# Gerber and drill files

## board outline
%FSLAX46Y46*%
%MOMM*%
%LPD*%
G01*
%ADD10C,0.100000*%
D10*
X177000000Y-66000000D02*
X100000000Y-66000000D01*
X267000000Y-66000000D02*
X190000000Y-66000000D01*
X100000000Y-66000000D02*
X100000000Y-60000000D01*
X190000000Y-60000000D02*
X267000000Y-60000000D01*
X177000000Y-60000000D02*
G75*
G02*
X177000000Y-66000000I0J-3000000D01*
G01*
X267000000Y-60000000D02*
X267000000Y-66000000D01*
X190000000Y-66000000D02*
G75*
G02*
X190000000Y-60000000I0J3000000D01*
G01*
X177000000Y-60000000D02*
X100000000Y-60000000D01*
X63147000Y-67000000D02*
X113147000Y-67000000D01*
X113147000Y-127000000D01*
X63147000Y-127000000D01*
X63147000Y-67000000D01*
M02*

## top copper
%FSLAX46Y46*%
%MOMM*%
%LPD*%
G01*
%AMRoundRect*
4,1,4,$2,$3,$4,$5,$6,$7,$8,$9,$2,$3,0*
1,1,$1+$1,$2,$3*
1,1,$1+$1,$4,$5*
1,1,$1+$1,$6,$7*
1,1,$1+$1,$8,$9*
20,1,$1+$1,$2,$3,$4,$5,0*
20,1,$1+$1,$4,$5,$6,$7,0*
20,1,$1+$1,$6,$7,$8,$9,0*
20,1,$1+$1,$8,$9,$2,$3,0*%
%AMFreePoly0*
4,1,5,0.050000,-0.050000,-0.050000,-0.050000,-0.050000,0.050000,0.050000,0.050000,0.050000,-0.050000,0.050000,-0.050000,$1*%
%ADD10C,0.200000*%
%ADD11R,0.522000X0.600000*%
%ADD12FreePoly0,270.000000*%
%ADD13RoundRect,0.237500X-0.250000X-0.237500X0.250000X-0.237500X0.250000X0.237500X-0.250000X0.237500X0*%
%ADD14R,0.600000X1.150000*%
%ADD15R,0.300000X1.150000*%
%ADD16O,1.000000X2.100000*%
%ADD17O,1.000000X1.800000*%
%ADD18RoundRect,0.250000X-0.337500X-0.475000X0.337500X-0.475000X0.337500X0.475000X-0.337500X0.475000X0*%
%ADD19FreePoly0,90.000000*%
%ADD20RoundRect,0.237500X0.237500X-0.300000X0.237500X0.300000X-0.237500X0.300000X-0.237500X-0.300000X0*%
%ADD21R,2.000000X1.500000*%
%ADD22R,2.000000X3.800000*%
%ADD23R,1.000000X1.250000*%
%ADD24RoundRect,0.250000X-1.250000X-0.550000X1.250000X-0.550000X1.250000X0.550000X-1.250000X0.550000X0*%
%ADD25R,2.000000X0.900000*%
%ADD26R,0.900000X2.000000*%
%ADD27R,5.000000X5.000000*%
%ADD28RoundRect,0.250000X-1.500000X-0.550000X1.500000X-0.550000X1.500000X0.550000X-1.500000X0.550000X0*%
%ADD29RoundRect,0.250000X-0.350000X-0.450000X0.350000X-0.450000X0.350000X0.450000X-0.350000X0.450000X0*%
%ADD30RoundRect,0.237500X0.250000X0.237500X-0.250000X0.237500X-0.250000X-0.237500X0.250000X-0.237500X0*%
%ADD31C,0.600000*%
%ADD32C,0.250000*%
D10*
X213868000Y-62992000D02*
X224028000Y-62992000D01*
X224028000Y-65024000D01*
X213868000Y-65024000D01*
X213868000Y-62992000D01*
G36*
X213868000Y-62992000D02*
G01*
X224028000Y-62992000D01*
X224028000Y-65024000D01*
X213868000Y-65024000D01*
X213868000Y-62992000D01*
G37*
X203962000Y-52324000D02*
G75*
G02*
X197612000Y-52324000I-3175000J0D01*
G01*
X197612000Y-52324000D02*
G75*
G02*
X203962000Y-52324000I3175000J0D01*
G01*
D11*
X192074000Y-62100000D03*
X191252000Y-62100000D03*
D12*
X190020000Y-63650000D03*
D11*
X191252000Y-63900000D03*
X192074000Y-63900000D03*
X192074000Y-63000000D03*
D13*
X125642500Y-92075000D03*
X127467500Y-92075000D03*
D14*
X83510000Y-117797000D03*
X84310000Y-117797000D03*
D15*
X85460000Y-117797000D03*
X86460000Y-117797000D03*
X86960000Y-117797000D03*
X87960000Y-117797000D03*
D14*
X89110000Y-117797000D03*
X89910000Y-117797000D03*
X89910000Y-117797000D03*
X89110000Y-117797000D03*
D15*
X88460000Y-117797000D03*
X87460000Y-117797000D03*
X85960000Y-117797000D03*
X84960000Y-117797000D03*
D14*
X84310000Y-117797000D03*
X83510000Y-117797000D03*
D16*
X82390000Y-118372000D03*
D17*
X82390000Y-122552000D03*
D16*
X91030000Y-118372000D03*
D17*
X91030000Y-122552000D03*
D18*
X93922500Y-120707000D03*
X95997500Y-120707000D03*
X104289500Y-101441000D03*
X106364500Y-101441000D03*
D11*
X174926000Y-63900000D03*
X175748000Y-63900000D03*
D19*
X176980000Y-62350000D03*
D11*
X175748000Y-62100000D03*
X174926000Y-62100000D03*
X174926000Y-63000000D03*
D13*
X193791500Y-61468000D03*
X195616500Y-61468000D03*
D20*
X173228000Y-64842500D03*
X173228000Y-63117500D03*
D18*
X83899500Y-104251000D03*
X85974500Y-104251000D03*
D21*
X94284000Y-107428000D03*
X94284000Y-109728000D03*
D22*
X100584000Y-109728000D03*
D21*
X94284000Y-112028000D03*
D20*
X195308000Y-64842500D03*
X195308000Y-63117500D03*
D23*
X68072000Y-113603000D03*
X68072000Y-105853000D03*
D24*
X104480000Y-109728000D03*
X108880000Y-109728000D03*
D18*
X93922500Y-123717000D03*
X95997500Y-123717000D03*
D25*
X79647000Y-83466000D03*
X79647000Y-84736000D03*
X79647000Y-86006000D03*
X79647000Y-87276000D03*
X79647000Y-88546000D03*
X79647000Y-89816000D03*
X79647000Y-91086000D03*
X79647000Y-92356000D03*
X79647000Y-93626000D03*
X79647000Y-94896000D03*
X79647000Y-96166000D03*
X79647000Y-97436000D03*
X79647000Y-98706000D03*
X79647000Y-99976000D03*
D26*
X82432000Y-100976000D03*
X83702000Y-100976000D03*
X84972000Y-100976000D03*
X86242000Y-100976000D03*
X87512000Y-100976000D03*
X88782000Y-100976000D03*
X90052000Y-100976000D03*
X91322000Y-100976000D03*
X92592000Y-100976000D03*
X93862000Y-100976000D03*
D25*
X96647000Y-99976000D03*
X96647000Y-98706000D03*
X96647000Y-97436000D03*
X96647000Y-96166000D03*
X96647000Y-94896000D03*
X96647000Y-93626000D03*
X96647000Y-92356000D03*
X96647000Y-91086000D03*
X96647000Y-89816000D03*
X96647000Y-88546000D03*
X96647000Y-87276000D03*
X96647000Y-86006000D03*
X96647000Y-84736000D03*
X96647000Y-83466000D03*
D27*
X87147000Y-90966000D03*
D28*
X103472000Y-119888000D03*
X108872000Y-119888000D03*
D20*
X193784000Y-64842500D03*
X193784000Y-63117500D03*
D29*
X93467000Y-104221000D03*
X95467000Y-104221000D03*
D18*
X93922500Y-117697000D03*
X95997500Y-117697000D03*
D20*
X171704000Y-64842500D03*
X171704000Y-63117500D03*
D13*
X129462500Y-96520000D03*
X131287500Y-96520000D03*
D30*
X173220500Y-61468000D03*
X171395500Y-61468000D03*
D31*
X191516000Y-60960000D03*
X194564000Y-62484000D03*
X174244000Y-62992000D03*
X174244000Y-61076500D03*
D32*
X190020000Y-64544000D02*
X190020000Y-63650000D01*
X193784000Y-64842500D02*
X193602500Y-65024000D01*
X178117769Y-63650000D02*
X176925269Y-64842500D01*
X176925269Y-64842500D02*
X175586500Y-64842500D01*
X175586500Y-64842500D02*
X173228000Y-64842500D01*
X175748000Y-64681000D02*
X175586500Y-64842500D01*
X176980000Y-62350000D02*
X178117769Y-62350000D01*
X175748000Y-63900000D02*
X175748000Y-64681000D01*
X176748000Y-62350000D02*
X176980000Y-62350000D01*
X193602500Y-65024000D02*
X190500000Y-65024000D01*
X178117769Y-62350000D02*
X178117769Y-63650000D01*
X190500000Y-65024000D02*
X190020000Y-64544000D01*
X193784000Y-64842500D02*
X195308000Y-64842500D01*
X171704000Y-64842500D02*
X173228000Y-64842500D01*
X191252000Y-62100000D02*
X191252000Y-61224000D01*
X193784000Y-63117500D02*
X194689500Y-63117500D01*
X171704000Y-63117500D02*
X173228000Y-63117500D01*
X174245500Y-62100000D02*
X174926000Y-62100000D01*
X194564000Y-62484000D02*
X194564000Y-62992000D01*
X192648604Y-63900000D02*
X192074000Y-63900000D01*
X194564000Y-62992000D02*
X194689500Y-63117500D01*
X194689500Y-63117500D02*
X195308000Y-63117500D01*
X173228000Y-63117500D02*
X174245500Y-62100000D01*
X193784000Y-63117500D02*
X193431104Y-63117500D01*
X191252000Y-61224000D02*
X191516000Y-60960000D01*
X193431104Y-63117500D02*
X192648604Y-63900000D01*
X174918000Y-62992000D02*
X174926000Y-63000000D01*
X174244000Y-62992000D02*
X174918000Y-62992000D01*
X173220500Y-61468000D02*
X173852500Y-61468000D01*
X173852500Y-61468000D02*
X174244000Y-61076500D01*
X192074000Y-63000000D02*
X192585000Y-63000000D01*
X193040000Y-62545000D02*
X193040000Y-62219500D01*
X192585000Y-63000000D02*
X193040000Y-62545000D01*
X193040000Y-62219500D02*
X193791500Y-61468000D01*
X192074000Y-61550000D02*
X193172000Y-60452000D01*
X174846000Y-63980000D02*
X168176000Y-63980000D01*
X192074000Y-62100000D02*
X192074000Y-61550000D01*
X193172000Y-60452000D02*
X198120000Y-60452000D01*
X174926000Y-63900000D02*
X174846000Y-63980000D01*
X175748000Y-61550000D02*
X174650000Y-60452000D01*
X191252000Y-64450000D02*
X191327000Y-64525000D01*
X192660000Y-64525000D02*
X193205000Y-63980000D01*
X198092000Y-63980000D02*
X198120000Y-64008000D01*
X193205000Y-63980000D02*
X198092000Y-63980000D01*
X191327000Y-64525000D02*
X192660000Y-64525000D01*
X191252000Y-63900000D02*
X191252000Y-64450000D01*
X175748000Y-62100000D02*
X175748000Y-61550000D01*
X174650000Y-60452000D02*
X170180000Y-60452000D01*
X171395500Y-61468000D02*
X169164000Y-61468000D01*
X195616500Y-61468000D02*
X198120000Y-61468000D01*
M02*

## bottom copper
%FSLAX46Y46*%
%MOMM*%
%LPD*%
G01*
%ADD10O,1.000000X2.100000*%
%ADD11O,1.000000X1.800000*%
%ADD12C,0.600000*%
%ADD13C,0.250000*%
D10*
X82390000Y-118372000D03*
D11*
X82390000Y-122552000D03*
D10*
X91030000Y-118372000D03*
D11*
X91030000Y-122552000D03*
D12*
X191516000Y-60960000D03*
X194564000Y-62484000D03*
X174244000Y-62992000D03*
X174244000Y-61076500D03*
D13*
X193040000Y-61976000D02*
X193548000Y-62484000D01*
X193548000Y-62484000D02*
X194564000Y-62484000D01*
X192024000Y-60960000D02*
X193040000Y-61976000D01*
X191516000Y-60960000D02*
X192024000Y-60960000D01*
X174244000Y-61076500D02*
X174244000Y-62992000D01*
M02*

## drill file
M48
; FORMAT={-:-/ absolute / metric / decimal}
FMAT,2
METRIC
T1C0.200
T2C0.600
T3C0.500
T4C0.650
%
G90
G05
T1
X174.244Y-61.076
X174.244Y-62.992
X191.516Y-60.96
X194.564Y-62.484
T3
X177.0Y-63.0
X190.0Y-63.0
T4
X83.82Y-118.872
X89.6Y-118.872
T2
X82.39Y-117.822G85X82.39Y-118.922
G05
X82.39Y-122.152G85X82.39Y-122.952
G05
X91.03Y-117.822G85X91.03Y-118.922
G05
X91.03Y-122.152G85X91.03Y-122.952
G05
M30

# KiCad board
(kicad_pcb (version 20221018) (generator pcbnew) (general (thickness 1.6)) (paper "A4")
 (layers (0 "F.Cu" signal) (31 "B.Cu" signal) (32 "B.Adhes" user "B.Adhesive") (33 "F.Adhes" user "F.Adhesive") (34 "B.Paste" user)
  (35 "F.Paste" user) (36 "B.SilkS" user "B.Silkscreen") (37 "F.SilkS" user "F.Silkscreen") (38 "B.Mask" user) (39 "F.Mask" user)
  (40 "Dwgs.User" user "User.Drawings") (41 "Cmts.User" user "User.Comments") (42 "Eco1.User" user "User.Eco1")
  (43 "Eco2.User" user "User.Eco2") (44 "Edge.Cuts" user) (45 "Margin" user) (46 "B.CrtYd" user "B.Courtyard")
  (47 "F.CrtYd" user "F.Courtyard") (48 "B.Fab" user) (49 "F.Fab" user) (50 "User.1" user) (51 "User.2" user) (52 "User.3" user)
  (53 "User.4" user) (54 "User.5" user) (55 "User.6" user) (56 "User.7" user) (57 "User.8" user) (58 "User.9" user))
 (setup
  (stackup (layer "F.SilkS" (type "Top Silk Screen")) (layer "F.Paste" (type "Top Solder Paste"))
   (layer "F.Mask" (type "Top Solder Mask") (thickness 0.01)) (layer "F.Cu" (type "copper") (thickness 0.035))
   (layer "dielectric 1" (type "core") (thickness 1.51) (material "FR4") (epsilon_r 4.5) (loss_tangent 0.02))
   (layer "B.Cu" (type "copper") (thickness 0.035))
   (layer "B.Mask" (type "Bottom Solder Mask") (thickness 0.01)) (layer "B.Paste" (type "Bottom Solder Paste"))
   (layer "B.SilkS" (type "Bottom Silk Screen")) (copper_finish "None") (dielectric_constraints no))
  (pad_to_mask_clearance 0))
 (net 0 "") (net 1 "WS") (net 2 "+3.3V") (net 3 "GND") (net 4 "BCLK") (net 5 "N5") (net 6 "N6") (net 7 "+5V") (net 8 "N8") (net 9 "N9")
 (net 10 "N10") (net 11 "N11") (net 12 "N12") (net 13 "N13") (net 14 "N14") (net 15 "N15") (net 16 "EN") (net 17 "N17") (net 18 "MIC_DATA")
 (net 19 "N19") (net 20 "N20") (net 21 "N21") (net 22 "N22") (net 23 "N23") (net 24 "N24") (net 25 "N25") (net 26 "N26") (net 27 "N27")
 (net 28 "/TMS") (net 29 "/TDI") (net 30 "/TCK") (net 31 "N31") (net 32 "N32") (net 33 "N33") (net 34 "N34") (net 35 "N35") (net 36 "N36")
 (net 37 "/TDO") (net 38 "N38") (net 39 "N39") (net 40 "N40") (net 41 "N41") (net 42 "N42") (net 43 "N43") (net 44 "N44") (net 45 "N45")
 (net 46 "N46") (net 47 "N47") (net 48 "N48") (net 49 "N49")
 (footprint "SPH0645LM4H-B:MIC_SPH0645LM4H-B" (layer "F.Cu") (at 190 63 -90)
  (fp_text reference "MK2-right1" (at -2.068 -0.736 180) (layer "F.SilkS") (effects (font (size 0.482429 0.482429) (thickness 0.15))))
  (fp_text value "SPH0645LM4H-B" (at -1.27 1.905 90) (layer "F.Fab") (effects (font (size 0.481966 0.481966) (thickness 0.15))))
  (pad "" np_thru_hole circle (at 0 0 270) (size 0.5 0.5) (drill 0.5) (layers "*.Cu" "*.Mask"))
  (pad "1" smd rect (at -0.9 -2.074 270) (size 0.6 0.522) (layers "F.Cu" "F.Paste" "F.Mask") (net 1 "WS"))
  (pad "2" smd rect (at -0.9 -1.252 270) (size 0.6 0.522) (layers "F.Cu" "F.Paste" "F.Mask") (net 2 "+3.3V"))
  (pad "3" smd custom (at 0.65 -0.02 270) (size 0.1 0.1) (layers "F.Cu") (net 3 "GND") (zone_connect 0) (thermal_bridge_angle 45)
   (options (clearance outline) (anchor rect)) (primitives))
  (pad "4" smd rect (at 0.9 -1.252 270) (size 0.6 0.522) (layers "F.Cu" "F.Paste" "F.Mask") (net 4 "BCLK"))
  (pad "5" smd rect (at 0.9 -2.074 270) (size 0.6 0.522) (layers "F.Cu" "F.Paste" "F.Mask") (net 2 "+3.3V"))
  (pad "6" smd rect (at 0 -2.074 270) (size 0.6 0.522) (layers "F.Cu" "F.Paste" "F.Mask") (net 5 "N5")))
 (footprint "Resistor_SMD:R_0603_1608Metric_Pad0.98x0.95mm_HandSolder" (layer "F.Cu") (at 126.555 92.075)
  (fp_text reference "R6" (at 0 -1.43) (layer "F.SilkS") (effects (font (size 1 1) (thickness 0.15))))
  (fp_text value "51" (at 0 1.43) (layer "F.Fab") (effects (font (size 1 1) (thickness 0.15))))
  (pad "1" smd roundrect (at -0.9125 0) (size 0.975 0.95) (layers "F.Cu" "F.Paste" "F.Mask") (roundrect_rratio 0.25) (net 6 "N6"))
  (pad "2" smd roundrect (at 0.9125 0) (size 0.975 0.95) (layers "F.Cu" "F.Paste" "F.Mask") (roundrect_rratio 0.25) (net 1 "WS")))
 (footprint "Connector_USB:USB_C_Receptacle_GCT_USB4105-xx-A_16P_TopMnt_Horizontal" (layer "F.Cu") (at 86.71 121.477)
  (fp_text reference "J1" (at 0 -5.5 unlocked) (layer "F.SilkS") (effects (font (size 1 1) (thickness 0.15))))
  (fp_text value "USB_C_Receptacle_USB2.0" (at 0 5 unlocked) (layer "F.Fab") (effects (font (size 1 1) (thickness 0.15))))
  (pad "" np_thru_hole circle (at -2.89 -2.605) (size 0.65 0.65) (drill 0.65) (layers "F&B.Cu" "*.Mask"))
  (pad "" np_thru_hole circle (at 2.89 -2.605) (size 0.65 0.65) (drill 0.65) (layers "F&B.Cu" "*.Mask"))
  (pad "A1" smd rect (at -3.2 -3.68) (size 0.6 1.15) (layers "F.Cu" "F.Paste" "F.Mask") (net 3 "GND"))
  (pad "A4" smd rect (at -2.4 -3.68) (size 0.6 1.15) (layers "F.Cu" "F.Paste" "F.Mask") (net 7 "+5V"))
  (pad "A5" smd rect (at -1.25 -3.68) (size 0.3 1.15) (layers "F.Cu" "F.Paste" "F.Mask") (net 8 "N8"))
  (pad "A6" smd rect (at -0.25 -3.68) (size 0.3 1.15) (layers "F.Cu" "F.Paste" "F.Mask") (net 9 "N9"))
  (pad "A7" smd rect (at 0.25 -3.68) (size 0.3 1.15) (layers "F.Cu" "F.Paste" "F.Mask") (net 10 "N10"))
  (pad "A8" smd rect (at 1.25 -3.68) (size 0.3 1.15) (layers "F.Cu" "F.Paste" "F.Mask") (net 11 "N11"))
  (pad "A9" smd rect (at 2.4 -3.68) (size 0.6 1.15) (layers "F.Cu" "F.Paste" "F.Mask") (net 7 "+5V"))
  (pad "A12" smd rect (at 3.2 -3.68) (size 0.6 1.15) (layers "F.Cu" "F.Paste" "F.Mask") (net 3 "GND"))
  (pad "B1" smd rect (at 3.2 -3.68) (size 0.6 1.15) (layers "F.Cu" "F.Paste" "F.Mask") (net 3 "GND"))
  (pad "B4" smd rect (at 2.4 -3.68) (size 0.6 1.15) (layers "F.Cu" "F.Paste" "F.Mask") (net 7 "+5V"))
  (pad "B5" smd rect (at 1.75 -3.68) (size 0.3 1.15) (layers "F.Cu" "F.Paste" "F.Mask") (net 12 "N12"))
  (pad "B6" smd rect (at 0.75 -3.68) (size 0.3 1.15) (layers "F.Cu" "F.Paste" "F.Mask") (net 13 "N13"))
  (pad "B7" smd rect (at -0.75 -3.68) (size 0.3 1.15) (layers "F.Cu" "F.Paste" "F.Mask") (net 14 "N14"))
  (pad "B8" smd rect (at -1.75 -3.68) (size 0.3 1.15) (layers "F.Cu" "F.Paste" "F.Mask") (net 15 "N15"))
  (pad "B9" smd rect (at -2.4 -3.68) (size 0.6 1.15) (layers "F.Cu" "F.Paste" "F.Mask") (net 7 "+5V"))
  (pad "B12" smd rect (at -3.2 -3.68) (size 0.6 1.15) (layers "F.Cu" "F.Paste" "F.Mask") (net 3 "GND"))
  (pad "S1" thru_hole oval (at -4.32 -3.105) (size 1 2.1) (drill oval 0.6 1.7) (layers "*.Cu" "*.Mask") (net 3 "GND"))
  (pad "S1" thru_hole oval (at -4.32 1.075) (size 1 1.8) (drill oval 0.6 1.4) (layers "*.Cu" "*.Mask") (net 3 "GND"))
  (pad "S1" thru_hole oval (at 4.32 -3.105) (size 1 2.1) (drill oval 0.6 1.7) (layers "*.Cu" "*.Mask") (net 3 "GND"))
  (pad "S1" thru_hole oval (at 4.32 1.075) (size 1 1.8) (drill oval 0.6 1.4) (layers "*.Cu" "*.Mask") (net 3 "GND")))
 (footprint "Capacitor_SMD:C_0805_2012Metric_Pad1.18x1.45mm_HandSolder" (layer "F.Cu") (at 94.96 120.707)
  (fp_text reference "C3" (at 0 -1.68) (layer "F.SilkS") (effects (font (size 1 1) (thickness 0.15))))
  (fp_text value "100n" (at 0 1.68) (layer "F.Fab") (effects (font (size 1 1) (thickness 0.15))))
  (pad "1" smd roundrect (at -1.0375 0) (size 1.175 1.45) (layers "F.Cu" "F.Paste" "F.Mask") (roundrect_rratio 0.212766) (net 3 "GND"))
  (pad "2" smd roundrect (at 1.0375 0) (size 1.175 1.45) (layers "F.Cu" "F.Paste" "F.Mask") (roundrect_rratio 0.212766) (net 2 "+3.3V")))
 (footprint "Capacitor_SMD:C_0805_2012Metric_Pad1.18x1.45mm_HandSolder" (layer "F.Cu") (at 105.327 101.441)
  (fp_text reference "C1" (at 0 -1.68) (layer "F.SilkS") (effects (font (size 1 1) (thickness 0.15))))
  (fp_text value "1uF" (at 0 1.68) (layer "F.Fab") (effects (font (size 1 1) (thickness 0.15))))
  (pad "1" smd roundrect (at -1.0375 0) (size 1.175 1.45) (layers "F.Cu" "F.Paste" "F.Mask") (roundrect_rratio 0.212766) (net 3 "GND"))
  (pad "2" smd roundrect (at 1.0375 0) (size 1.175 1.45) (layers "F.Cu" "F.Paste" "F.Mask") (roundrect_rratio 0.212766) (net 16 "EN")))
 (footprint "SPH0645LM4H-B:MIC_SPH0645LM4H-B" (layer "F.Cu") (at 177 63 90)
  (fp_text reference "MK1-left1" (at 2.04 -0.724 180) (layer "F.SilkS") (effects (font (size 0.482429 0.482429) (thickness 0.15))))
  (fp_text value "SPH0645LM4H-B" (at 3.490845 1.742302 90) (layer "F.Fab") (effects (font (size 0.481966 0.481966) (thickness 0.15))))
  (pad "" np_thru_hole circle (at 0 0 90) (size 0.5 0.5) (drill 0.5) (layers "*.Cu" "*.Mask"))
  (pad "1" smd rect (at -0.9 -2.074 90) (size 0.6 0.522) (layers "F.Cu" "F.Paste" "F.Mask") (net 1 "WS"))
  (pad "2" smd rect (at -0.9 -1.252 90) (size 0.6 0.522) (layers "F.Cu" "F.Paste" "F.Mask") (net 3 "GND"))
  (pad "3" smd custom (at 0.65 -0.02 90) (size 0.1 0.1) (layers "F.Cu") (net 3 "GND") (zone_connect 0) (thermal_bridge_angle 45)
   (options (clearance outline) (anchor rect)) (primitives))
  (pad "4" smd rect (at 0.9 -1.252 90) (size 0.6 0.522) (layers "F.Cu" "F.Paste" "F.Mask") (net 4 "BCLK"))
  (pad "5" smd rect (at 0.9 -2.074 90) (size 0.6 0.522) (layers "F.Cu" "F.Paste" "F.Mask") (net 2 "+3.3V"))
  (pad "6" smd rect (at 0 -2.074 90) (size 0.6 0.522) (layers "F.Cu" "F.Paste" "F.Mask") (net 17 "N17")))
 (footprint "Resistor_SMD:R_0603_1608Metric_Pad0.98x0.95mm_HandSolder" (layer "F.Cu") (at 194.704 61.468)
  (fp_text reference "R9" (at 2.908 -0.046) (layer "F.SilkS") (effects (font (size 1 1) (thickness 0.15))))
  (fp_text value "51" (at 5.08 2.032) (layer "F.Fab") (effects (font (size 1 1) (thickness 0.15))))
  (pad "1" smd roundrect (at -0.9125 0) (size 0.975 0.95) (layers "F.Cu" "F.Paste" "F.Mask") (roundrect_rratio 0.25) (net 5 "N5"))
  (pad "2" smd roundrect (at 0.9125 0) (size 0.975 0.95) (layers "F.Cu" "F.Paste" "F.Mask") (roundrect_rratio 0.25) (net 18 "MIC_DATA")))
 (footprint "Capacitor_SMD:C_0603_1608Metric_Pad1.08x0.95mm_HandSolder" (layer "F.Cu") (at 173.228 63.98 90)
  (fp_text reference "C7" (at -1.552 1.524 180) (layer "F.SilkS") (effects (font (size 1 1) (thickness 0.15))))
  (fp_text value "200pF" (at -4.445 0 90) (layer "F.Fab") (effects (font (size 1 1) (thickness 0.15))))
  (pad "1" smd roundrect (at -0.8625 0 90) (size 1.075 0.95) (layers "F.Cu" "F.Paste" "F.Mask") (roundrect_rratio 0.25) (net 3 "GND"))
  (pad "2" smd roundrect (at 0.8625 0 90) (size 1.075 0.95) (layers "F.Cu" "F.Paste" "F.Mask") (roundrect_rratio 0.25) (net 2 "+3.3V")))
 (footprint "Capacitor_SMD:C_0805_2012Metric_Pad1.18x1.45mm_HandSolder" (layer "F.Cu") (at 84.937 104.251)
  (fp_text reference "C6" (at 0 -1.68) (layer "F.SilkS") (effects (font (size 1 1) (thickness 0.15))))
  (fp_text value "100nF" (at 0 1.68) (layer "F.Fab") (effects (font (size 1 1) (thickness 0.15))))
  (pad "1" smd roundrect (at -1.0375 0) (size 1.175 1.45) (layers "F.Cu" "F.Paste" "F.Mask") (roundrect_rratio 0.212766) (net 2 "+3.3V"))
  (pad "2" smd roundrect (at 1.0375 0) (size 1.175 1.45) (layers "F.Cu" "F.Paste" "F.Mask") (roundrect_rratio 0.212766) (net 3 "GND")))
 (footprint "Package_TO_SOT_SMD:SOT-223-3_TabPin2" (layer "F.Cu") (at 97.434 109.728)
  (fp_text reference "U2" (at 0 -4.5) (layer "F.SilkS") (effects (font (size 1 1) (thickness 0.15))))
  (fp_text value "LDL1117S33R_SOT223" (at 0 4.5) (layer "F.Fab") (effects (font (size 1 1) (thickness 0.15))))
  (pad "1" smd rect (at -3.15 -2.3) (size 2 1.5) (layers "F.Cu" "F.Paste" "F.Mask") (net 3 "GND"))
  (pad "2" smd rect (at -3.15 0) (size 2 1.5) (layers "F.Cu" "F.Paste" "F.Mask") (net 2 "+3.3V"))
  (pad "2" smd rect (at 3.15 0) (size 2 3.8) (layers "F.Cu" "F.Paste" "F.Mask") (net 2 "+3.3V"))
  (pad "3" smd rect (at -3.15 2.3) (size 2 1.5) (layers "F.Cu" "F.Paste" "F.Mask") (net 7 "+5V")))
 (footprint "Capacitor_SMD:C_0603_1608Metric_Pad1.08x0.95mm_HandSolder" (layer "F.Cu") (at 195.308 63.98 90)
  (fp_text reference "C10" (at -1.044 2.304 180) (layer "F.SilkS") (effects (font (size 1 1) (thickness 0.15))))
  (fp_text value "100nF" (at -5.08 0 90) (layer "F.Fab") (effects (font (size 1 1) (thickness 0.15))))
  (pad "1" smd roundrect (at -0.8625 0 90) (size 1.075 0.95) (layers "F.Cu" "F.Paste" "F.Mask") (roundrect_rratio 0.25) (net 3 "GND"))
  (pad "2" smd roundrect (at 0.8625 0 90) (size 1.075 0.95) (layers "F.Cu" "F.Paste" "F.Mask") (roundrect_rratio 0.25) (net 2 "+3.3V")))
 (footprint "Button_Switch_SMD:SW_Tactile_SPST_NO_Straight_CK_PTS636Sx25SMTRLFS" (layer "F.Cu") (at 68.072 109.728 90)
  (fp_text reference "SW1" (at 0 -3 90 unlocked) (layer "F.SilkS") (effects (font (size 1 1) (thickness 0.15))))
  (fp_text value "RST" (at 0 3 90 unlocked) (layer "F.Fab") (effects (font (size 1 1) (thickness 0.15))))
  (pad "1" smd rect (at -3.875 0 90) (size 1.25 1) (layers "F.Cu" "F.Paste" "F.Mask") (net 3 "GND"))
  (pad "2" smd rect (at 3.875 0 90) (size 1.25 1) (layers "F.Cu" "F.Paste" "F.Mask") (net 16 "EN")))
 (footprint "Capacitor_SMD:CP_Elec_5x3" (layer "F.Cu") (at 106.68 109.728)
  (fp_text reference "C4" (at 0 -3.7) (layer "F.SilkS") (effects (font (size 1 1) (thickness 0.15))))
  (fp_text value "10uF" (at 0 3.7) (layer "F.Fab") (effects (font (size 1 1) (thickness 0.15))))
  (pad "1" smd roundrect (at -2.2 0) (size 3 1.6) (layers "F.Cu" "F.Paste" "F.Mask") (roundrect_rratio 0.15625) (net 7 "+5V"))
  (pad "2" smd roundrect (at 2.2 0) (size 3 1.6) (layers "F.Cu" "F.Paste" "F.Mask") (roundrect_rratio 0.15625) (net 3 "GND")))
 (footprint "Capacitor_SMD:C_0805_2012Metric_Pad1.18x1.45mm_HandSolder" (layer "F.Cu") (at 94.96 123.717)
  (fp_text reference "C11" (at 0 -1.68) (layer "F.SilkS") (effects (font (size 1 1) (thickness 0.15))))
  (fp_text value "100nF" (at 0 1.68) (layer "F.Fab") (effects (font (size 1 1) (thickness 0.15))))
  (pad "1" smd roundrect (at -1.0375 0) (size 1.175 1.45) (layers "F.Cu" "F.Paste" "F.Mask") (roundrect_rratio 0.212766) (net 3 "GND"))
  (pad "2" smd roundrect (at 1.0375 0) (size 1.175 1.45) (layers "F.Cu" "F.Paste" "F.Mask") (roundrect_rratio 0.212766) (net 16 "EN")))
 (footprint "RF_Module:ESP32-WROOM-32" (layer "F.Cu") (at 88.147 91.721)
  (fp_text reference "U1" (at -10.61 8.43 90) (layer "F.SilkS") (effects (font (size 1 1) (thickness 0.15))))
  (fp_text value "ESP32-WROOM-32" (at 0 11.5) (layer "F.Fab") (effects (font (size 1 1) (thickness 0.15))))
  (pad "1" smd rect (at -8.5 -8.255) (size 2 0.9) (layers "F.Cu" "F.Paste" "F.Mask") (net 3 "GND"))
  (pad "2" smd rect (at -8.5 -6.985) (size 2 0.9) (layers "F.Cu" "F.Paste" "F.Mask") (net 2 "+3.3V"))
  (pad "3" smd rect (at -8.5 -5.715) (size 2 0.9) (layers "F.Cu" "F.Paste" "F.Mask") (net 16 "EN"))
  (pad "4" smd rect (at -8.5 -4.445) (size 2 0.9) (layers "F.Cu" "F.Paste" "F.Mask") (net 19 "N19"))
  (pad "5" smd rect (at -8.5 -3.175) (size 2 0.9) (layers "F.Cu" "F.Paste" "F.Mask") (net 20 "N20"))
  (pad "6" smd rect (at -8.5 -1.905) (size 2 0.9) (layers "F.Cu" "F.Paste" "F.Mask") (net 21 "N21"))
  (pad "7" smd rect (at -8.5 -0.635) (size 2 0.9) (layers "F.Cu" "F.Paste" "F.Mask") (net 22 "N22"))
  (pad "8" smd rect (at -8.5 0.635) (size 2 0.9) (layers "F.Cu" "F.Paste" "F.Mask") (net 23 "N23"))
  (pad "9" smd rect (at -8.5 1.905) (size 2 0.9) (layers "F.Cu" "F.Paste" "F.Mask") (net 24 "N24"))
  (pad "10" smd rect (at -8.5 3.175) (size 2 0.9) (layers "F.Cu" "F.Paste" "F.Mask") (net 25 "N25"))
  (pad "11" smd rect (at -8.5 4.445) (size 2 0.9) (layers "F.Cu" "F.Paste" "F.Mask") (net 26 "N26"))
  (pad "12" smd rect (at -8.5 5.715) (size 2 0.9) (layers "F.Cu" "F.Paste" "F.Mask") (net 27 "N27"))
  (pad "13" smd rect (at -8.5 6.985) (size 2 0.9) (layers "F.Cu" "F.Paste" "F.Mask") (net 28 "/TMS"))
  (pad "14" smd rect (at -8.5 8.255) (size 2 0.9) (layers "F.Cu" "F.Paste" "F.Mask") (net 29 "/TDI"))
  (pad "15" smd rect (at -5.715 9.255 90) (size 2 0.9) (layers "F.Cu" "F.Paste" "F.Mask") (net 3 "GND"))
  (pad "16" smd rect (at -4.445 9.255 90) (size 2 0.9) (layers "F.Cu" "F.Paste" "F.Mask") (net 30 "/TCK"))
  (pad "17" smd rect (at -3.175 9.255 90) (size 2 0.9) (layers "F.Cu" "F.Paste" "F.Mask") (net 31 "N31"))
  (pad "18" smd rect (at -1.905 9.255 90) (size 2 0.9) (layers "F.Cu" "F.Paste" "F.Mask") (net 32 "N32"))
  (pad "19" smd rect (at -0.635 9.255 90) (size 2 0.9) (layers "F.Cu" "F.Paste" "F.Mask") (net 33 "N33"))
  (pad "20" smd rect (at 0.635 9.255 90) (size 2 0.9) (layers "F.Cu" "F.Paste" "F.Mask") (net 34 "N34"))
  (pad "21" smd rect (at 1.905 9.255 90) (size 2 0.9) (layers "F.Cu" "F.Paste" "F.Mask") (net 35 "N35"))
  (pad "22" smd rect (at 3.175 9.255 90) (size 2 0.9) (layers "F.Cu" "F.Paste" "F.Mask") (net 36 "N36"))
  (pad "23" smd rect (at 4.445 9.255 90) (size 2 0.9) (layers "F.Cu" "F.Paste" "F.Mask") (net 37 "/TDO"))
  (pad "24" smd rect (at 5.715 9.255 90) (size 2 0.9) (layers "F.Cu" "F.Paste" "F.Mask") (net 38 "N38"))
  (pad "25" smd rect (at 8.5 8.255) (size 2 0.9) (layers "F.Cu" "F.Paste" "F.Mask") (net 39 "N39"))
  (pad "26" smd rect (at 8.5 6.985) (size 2 0.9) (layers "F.Cu" "F.Paste" "F.Mask") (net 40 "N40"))
  (pad "27" smd rect (at 8.5 5.715) (size 2 0.9) (layers "F.Cu" "F.Paste" "F.Mask") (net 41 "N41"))
  (pad "28" smd rect (at 8.5 4.445) (size 2 0.9) (layers "F.Cu" "F.Paste" "F.Mask") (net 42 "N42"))
  (pad "29" smd rect (at 8.5 3.175) (size 2 0.9) (layers "F.Cu" "F.Paste" "F.Mask") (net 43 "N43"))
  (pad "30" smd rect (at 8.5 1.905) (size 2 0.9) (layers "F.Cu" "F.Paste" "F.Mask") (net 6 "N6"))
  (pad "31" smd rect (at 8.5 0.635) (size 2 0.9) (layers "F.Cu" "F.Paste" "F.Mask") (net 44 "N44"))
  (pad "32" smd rect (at 8.5 -0.635) (size 2 0.9) (layers "F.Cu" "F.Paste" "F.Mask") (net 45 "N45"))
  (pad "33" smd rect (at 8.5 -1.905) (size 2 0.9) (layers "F.Cu" "F.Paste" "F.Mask") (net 18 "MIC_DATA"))
  (pad "34" smd rect (at 8.5 -3.175) (size 2 0.9) (layers "F.Cu" "F.Paste" "F.Mask") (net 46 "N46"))
  (pad "35" smd rect (at 8.5 -4.445) (size 2 0.9) (layers "F.Cu" "F.Paste" "F.Mask") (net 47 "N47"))
  (pad "36" smd rect (at 8.5 -5.715) (size 2 0.9) (layers "F.Cu" "F.Paste" "F.Mask") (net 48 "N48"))
  (pad "37" smd rect (at 8.5 -6.985) (size 2 0.9) (layers "F.Cu" "F.Paste" "F.Mask") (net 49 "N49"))
  (pad "38" smd rect (at 8.5 -8.255) (size 2 0.9) (layers "F.Cu" "F.Paste" "F.Mask") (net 3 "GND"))
  (pad "39" smd rect (at -1 -0.755) (size 5 5) (layers "F.Cu" "F.Paste" "F.Mask") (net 3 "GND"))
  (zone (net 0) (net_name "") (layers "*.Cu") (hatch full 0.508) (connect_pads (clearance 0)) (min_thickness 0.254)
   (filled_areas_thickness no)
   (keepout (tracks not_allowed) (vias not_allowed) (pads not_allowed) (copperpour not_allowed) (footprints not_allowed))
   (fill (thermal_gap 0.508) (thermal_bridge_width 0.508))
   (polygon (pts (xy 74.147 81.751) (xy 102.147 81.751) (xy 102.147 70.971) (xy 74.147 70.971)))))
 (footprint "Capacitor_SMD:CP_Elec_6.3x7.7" (layer "F.Cu") (at 106.172 119.888)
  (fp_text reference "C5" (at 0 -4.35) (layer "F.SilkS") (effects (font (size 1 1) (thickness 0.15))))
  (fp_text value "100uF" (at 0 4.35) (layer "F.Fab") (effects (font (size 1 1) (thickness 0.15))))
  (pad "1" smd roundrect (at -2.7 0) (size 3.5 1.6) (layers "F.Cu" "F.Paste" "F.Mask") (roundrect_rratio 0.15625) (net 2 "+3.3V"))
  (pad "2" smd roundrect (at 2.7 0) (size 3.5 1.6) (layers "F.Cu" "F.Paste" "F.Mask") (roundrect_rratio 0.15625) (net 3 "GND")))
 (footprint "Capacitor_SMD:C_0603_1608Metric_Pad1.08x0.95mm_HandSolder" (layer "F.Cu") (at 193.784 63.98 90)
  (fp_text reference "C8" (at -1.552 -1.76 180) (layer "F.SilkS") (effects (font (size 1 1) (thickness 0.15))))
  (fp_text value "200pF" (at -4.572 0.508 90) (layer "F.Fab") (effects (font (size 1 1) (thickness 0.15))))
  (pad "1" smd roundrect (at -0.8625 0 90) (size 1.075 0.95) (layers "F.Cu" "F.Paste" "F.Mask") (roundrect_rratio 0.25) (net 3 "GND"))
  (pad "2" smd roundrect (at 0.8625 0 90) (size 1.075 0.95) (layers "F.Cu" "F.Paste" "F.Mask") (roundrect_rratio 0.25) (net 2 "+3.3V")))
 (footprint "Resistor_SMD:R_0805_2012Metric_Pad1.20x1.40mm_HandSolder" (layer "F.Cu") (at 94.467 104.221)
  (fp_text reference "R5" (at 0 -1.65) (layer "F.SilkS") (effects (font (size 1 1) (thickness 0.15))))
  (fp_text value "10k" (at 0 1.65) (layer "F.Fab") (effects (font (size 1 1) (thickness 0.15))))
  (pad "1" smd roundrect (at -1 0) (size 1.2 1.4) (layers "F.Cu" "F.Paste" "F.Mask") (roundrect_rratio 0.208333) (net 2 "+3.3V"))
  (pad "2" smd roundrect (at 1 0) (size 1.2 1.4) (layers "F.Cu" "F.Paste" "F.Mask") (roundrect_rratio 0.208333) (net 16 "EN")))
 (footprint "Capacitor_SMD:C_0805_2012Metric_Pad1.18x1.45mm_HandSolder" (layer "F.Cu") (at 94.96 117.697)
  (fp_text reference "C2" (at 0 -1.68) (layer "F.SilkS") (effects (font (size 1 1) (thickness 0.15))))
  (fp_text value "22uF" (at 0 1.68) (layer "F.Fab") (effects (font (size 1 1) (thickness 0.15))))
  (pad "1" smd roundrect (at -1.0375 0) (size 1.175 1.45) (layers "F.Cu" "F.Paste" "F.Mask") (roundrect_rratio 0.212766) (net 3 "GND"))
  (pad "2" smd roundrect (at 1.0375 0) (size 1.175 1.45) (layers "F.Cu" "F.Paste" "F.Mask") (roundrect_rratio 0.212766) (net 2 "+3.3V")))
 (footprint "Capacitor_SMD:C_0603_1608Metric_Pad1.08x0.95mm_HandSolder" (layer "F.Cu") (at 171.704 63.98 90)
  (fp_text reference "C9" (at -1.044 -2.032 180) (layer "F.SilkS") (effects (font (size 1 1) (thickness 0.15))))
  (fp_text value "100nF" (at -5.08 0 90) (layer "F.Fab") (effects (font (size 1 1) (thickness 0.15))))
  (pad "1" smd roundrect (at -0.8625 0 90) (size 1.075 0.95) (layers "F.Cu" "F.Paste" "F.Mask") (roundrect_rratio 0.25) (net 3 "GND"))
  (pad "2" smd roundrect (at 0.8625 0 90) (size 1.075 0.95) (layers "F.Cu" "F.Paste" "F.Mask") (roundrect_rratio 0.25) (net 2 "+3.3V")))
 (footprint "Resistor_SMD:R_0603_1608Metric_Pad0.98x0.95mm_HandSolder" (layer "F.Cu") (at 130.375 96.52)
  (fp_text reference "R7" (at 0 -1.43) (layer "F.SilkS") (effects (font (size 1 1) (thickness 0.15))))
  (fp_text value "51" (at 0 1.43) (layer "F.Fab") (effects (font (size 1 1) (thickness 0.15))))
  (pad "1" smd roundrect (at -0.9125 0) (size 0.975 0.95) (layers "F.Cu" "F.Paste" "F.Mask") (roundrect_rratio 0.25) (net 44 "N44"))
  (pad "2" smd roundrect (at 0.9125 0) (size 0.975 0.95) (layers "F.Cu" "F.Paste" "F.Mask") (roundrect_rratio 0.25) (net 4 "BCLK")))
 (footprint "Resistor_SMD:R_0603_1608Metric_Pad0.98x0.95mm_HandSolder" (layer "F.Cu") (at 172.308 61.468 180)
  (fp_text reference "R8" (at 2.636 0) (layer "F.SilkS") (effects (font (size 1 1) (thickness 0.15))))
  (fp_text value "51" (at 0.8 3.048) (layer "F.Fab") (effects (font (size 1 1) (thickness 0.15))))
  (pad "1" smd roundrect (at -0.9125 0 180) (size 0.975 0.95) (layers "F.Cu" "F.Paste" "F.Mask") (roundrect_rratio 0.25) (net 17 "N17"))
  (pad "2" smd roundrect (at 0.9125 0 180) (size 0.975 0.95) (layers "F.Cu" "F.Paste" "F.Mask") (roundrect_rratio 0.25) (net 18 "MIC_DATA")))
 (gr_rect (start 213.868 62.992) (end 224.028 65.024) (stroke (width 0.2) (type solid)) (fill solid) (layer "F.Cu"))
 (gr_circle (center 200.787 52.324) (end 200.787 49.149) (stroke (width 0.2) (type solid)) (fill none) (layer "F.Cu"))
 (gr_line (start 177 66) (end 100 66) (stroke (width 0.1) (type solid)) (layer "Edge.Cuts"))
 (gr_line (start 267 66) (end 190 66) (stroke (width 0.1) (type solid)) (layer "Edge.Cuts"))
 (gr_line (start 100 66) (end 100 60) (stroke (width 0.1) (type solid)) (layer "Edge.Cuts"))
 (gr_line (start 190 60) (end 267 60) (stroke (width 0.1) (type solid)) (layer "Edge.Cuts"))
 (gr_arc (start 177 60) (mid 180 63) (end 177 66) (stroke (width 0.1) (type solid)) (layer "Edge.Cuts"))
 (gr_line (start 267 60) (end 267 66) (stroke (width 0.1) (type solid)) (layer "Edge.Cuts"))
 (gr_arc (start 190 66) (mid 187 63) (end 190 60) (stroke (width 0.1) (type solid)) (layer "Edge.Cuts"))
 (gr_line (start 177 60) (end 100 60) (stroke (width 0.1) (type solid)) (layer "Edge.Cuts"))
 (gr_rect (start 63.147 67) (end 113.147 127) (stroke (width 0.1) (type solid)) (fill none) (layer "Edge.Cuts"))
 (segment (start 190.02 64.544) (end 190.02 63.65) (width 0.25) (layer "F.Cu") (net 3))
 (segment (start 193.784 64.8425) (end 193.6025 65.024) (width 0.25) (layer "F.Cu") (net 3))
 (segment (start 178.117769 63.65) (end 176.925269 64.8425) (width 0.25) (layer "F.Cu") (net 3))
 (segment (start 176.925269 64.8425) (end 175.5865 64.8425) (width 0.25) (layer "F.Cu") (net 3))
 (segment (start 175.5865 64.8425) (end 173.228 64.8425) (width 0.25) (layer "F.Cu") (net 3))
 (segment (start 175.748 64.681) (end 175.5865 64.8425) (width 0.25) (layer "F.Cu") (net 3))
 (segment (start 176.98 62.35) (end 178.117769 62.35) (width 0.25) (layer "F.Cu") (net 3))
 (segment (start 175.748 63.9) (end 175.748 64.681) (width 0.25) (layer "F.Cu") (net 3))
 (segment (start 176.748 62.35) (end 176.98 62.35) (width 0.25) (layer "F.Cu") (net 3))
 (segment (start 193.6025 65.024) (end 190.5 65.024) (width 0.25) (layer "F.Cu") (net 3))
 (segment (start 178.117769 62.35) (end 178.117769 63.65) (width 0.25) (layer "F.Cu") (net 3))
 (segment (start 190.5 65.024) (end 190.02 64.544) (width 0.25) (layer "F.Cu") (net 3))
 (segment (start 193.784 64.8425) (end 195.308 64.8425) (width 0.25) (layer "F.Cu") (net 3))
 (segment (start 171.704 64.8425) (end 173.228 64.8425) (width 0.25) (layer "F.Cu") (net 3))
 (segment (start 191.252 62.1) (end 191.252 61.224) (width 0.25) (layer "F.Cu") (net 2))
 (segment (start 193.784 63.1175) (end 194.6895 63.1175) (width 0.25) (layer "F.Cu") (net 2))
 (segment (start 171.704 63.1175) (end 173.228 63.1175) (width 0.25) (layer "F.Cu") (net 2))
 (segment (start 174.2455 62.1) (end 174.926 62.1) (width 0.25) (layer "F.Cu") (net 2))
 (segment (start 194.564 62.484) (end 194.564 62.992) (width 0.25) (layer "F.Cu") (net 2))
 (segment (start 192.648604 63.9) (end 192.074 63.9) (width 0.25) (layer "F.Cu") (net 2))
 (segment (start 194.564 62.992) (end 194.6895 63.1175) (width 0.25) (layer "F.Cu") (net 2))
 (segment (start 194.6895 63.1175) (end 195.308 63.1175) (width 0.25) (layer "F.Cu") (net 2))
 (segment (start 173.228 63.1175) (end 174.2455 62.1) (width 0.25) (layer "F.Cu") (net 2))
 (segment (start 193.784 63.1175) (end 193.431104 63.1175) (width 0.25) (layer "F.Cu") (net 2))
 (segment (start 191.252 61.224) (end 191.516 60.96) (width 0.25) (layer "F.Cu") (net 2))
 (segment (start 193.431104 63.1175) (end 192.648604 63.9) (width 0.25) (layer "F.Cu") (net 2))
 (via (at 191.516 60.96) (size 0.6) (drill 0.2) (layers "F.Cu" "B.Cu") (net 2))
 (via (at 194.564 62.484) (size 0.6) (drill 0.2) (layers "F.Cu" "B.Cu") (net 2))
 (segment (start 193.04 61.976) (end 193.548 62.484) (width 0.25) (layer "B.Cu") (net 2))
 (segment (start 193.548 62.484) (end 194.564 62.484) (width 0.25) (layer "B.Cu") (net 2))
 (segment (start 192.024 60.96) (end 193.04 61.976) (width 0.25) (layer "B.Cu") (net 2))
 (segment (start 191.516 60.96) (end 192.024 60.96) (width 0.25) (layer "B.Cu") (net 2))
 (segment (start 174.918 62.992) (end 174.926 63) (width 0.25) (layer "F.Cu") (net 17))
 (segment (start 174.244 62.992) (end 174.918 62.992) (width 0.25) (layer "F.Cu") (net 17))
 (segment (start 173.2205 61.468) (end 173.8525 61.468) (width 0.25) (layer "F.Cu") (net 17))
 (segment (start 173.8525 61.468) (end 174.244 61.0765) (width 0.25) (layer "F.Cu") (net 17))
 (via (at 174.244 62.992) (size 0.6) (drill 0.2) (layers "F.Cu" "B.Cu") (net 17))
 (via (at 174.244 61.0765) (size 0.6) (drill 0.2) (layers "F.Cu" "B.Cu") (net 17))
 (segment (start 174.244 61.0765) (end 174.244 62.992) (width 0.25) (layer "B.Cu") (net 17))
 (segment (start 192.074 63) (end 192.585 63) (width 0.25) (layer "F.Cu") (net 5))
 (segment (start 193.04 62.545) (end 193.04 62.2195) (width 0.25) (layer "F.Cu") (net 5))
 (segment (start 192.585 63) (end 193.04 62.545) (width 0.25) (layer "F.Cu") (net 5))
 (segment (start 193.04 62.2195) (end 193.7915 61.468) (width 0.25) (layer "F.Cu") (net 5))
 (segment (start 192.074 61.55) (end 193.172 60.452) (width 0.25) (layer "F.Cu") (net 1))
 (segment (start 174.846 63.98) (end 168.176 63.98) (width 0.25) (layer "F.Cu") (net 1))
 (segment (start 192.074 62.1) (end 192.074 61.55) (width 0.25) (layer "F.Cu") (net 1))
 (segment (start 193.172 60.452) (end 198.12 60.452) (width 0.25) (layer "F.Cu") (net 1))
 (segment (start 174.926 63.9) (end 174.846 63.98) (width 0.25) (layer "F.Cu") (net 1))
 (segment (start 175.748 61.55) (end 174.65 60.452) (width 0.25) (layer "F.Cu") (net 4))
 (segment (start 191.252 64.45) (end 191.327 64.525) (width 0.25) (layer "F.Cu") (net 4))
 (segment (start 192.66 64.525) (end 193.205 63.98) (width 0.25) (layer "F.Cu") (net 4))
 (segment (start 198.092 63.98) (end 198.12 64.008) (width 0.25) (layer "F.Cu") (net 4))
 (segment (start 193.205 63.98) (end 198.092 63.98) (width 0.25) (layer "F.Cu") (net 4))
 (segment (start 191.327 64.525) (end 192.66 64.525) (width 0.25) (layer "F.Cu") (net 4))
 (segment (start 191.252 63.9) (end 191.252 64.45) (width 0.25) (layer "F.Cu") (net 4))
 (segment (start 175.748 62.1) (end 175.748 61.55) (width 0.25) (layer "F.Cu") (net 4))
 (segment (start 174.65 60.452) (end 170.18 60.452) (width 0.25) (layer "F.Cu") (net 4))
 (segment (start 171.3955 61.468) (end 169.164 61.468) (width 0.25) (layer "F.Cu") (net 18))
 (segment (start 195.6165 61.468) (end 198.12 61.468) (width 0.25) (layer "F.Cu") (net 18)))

